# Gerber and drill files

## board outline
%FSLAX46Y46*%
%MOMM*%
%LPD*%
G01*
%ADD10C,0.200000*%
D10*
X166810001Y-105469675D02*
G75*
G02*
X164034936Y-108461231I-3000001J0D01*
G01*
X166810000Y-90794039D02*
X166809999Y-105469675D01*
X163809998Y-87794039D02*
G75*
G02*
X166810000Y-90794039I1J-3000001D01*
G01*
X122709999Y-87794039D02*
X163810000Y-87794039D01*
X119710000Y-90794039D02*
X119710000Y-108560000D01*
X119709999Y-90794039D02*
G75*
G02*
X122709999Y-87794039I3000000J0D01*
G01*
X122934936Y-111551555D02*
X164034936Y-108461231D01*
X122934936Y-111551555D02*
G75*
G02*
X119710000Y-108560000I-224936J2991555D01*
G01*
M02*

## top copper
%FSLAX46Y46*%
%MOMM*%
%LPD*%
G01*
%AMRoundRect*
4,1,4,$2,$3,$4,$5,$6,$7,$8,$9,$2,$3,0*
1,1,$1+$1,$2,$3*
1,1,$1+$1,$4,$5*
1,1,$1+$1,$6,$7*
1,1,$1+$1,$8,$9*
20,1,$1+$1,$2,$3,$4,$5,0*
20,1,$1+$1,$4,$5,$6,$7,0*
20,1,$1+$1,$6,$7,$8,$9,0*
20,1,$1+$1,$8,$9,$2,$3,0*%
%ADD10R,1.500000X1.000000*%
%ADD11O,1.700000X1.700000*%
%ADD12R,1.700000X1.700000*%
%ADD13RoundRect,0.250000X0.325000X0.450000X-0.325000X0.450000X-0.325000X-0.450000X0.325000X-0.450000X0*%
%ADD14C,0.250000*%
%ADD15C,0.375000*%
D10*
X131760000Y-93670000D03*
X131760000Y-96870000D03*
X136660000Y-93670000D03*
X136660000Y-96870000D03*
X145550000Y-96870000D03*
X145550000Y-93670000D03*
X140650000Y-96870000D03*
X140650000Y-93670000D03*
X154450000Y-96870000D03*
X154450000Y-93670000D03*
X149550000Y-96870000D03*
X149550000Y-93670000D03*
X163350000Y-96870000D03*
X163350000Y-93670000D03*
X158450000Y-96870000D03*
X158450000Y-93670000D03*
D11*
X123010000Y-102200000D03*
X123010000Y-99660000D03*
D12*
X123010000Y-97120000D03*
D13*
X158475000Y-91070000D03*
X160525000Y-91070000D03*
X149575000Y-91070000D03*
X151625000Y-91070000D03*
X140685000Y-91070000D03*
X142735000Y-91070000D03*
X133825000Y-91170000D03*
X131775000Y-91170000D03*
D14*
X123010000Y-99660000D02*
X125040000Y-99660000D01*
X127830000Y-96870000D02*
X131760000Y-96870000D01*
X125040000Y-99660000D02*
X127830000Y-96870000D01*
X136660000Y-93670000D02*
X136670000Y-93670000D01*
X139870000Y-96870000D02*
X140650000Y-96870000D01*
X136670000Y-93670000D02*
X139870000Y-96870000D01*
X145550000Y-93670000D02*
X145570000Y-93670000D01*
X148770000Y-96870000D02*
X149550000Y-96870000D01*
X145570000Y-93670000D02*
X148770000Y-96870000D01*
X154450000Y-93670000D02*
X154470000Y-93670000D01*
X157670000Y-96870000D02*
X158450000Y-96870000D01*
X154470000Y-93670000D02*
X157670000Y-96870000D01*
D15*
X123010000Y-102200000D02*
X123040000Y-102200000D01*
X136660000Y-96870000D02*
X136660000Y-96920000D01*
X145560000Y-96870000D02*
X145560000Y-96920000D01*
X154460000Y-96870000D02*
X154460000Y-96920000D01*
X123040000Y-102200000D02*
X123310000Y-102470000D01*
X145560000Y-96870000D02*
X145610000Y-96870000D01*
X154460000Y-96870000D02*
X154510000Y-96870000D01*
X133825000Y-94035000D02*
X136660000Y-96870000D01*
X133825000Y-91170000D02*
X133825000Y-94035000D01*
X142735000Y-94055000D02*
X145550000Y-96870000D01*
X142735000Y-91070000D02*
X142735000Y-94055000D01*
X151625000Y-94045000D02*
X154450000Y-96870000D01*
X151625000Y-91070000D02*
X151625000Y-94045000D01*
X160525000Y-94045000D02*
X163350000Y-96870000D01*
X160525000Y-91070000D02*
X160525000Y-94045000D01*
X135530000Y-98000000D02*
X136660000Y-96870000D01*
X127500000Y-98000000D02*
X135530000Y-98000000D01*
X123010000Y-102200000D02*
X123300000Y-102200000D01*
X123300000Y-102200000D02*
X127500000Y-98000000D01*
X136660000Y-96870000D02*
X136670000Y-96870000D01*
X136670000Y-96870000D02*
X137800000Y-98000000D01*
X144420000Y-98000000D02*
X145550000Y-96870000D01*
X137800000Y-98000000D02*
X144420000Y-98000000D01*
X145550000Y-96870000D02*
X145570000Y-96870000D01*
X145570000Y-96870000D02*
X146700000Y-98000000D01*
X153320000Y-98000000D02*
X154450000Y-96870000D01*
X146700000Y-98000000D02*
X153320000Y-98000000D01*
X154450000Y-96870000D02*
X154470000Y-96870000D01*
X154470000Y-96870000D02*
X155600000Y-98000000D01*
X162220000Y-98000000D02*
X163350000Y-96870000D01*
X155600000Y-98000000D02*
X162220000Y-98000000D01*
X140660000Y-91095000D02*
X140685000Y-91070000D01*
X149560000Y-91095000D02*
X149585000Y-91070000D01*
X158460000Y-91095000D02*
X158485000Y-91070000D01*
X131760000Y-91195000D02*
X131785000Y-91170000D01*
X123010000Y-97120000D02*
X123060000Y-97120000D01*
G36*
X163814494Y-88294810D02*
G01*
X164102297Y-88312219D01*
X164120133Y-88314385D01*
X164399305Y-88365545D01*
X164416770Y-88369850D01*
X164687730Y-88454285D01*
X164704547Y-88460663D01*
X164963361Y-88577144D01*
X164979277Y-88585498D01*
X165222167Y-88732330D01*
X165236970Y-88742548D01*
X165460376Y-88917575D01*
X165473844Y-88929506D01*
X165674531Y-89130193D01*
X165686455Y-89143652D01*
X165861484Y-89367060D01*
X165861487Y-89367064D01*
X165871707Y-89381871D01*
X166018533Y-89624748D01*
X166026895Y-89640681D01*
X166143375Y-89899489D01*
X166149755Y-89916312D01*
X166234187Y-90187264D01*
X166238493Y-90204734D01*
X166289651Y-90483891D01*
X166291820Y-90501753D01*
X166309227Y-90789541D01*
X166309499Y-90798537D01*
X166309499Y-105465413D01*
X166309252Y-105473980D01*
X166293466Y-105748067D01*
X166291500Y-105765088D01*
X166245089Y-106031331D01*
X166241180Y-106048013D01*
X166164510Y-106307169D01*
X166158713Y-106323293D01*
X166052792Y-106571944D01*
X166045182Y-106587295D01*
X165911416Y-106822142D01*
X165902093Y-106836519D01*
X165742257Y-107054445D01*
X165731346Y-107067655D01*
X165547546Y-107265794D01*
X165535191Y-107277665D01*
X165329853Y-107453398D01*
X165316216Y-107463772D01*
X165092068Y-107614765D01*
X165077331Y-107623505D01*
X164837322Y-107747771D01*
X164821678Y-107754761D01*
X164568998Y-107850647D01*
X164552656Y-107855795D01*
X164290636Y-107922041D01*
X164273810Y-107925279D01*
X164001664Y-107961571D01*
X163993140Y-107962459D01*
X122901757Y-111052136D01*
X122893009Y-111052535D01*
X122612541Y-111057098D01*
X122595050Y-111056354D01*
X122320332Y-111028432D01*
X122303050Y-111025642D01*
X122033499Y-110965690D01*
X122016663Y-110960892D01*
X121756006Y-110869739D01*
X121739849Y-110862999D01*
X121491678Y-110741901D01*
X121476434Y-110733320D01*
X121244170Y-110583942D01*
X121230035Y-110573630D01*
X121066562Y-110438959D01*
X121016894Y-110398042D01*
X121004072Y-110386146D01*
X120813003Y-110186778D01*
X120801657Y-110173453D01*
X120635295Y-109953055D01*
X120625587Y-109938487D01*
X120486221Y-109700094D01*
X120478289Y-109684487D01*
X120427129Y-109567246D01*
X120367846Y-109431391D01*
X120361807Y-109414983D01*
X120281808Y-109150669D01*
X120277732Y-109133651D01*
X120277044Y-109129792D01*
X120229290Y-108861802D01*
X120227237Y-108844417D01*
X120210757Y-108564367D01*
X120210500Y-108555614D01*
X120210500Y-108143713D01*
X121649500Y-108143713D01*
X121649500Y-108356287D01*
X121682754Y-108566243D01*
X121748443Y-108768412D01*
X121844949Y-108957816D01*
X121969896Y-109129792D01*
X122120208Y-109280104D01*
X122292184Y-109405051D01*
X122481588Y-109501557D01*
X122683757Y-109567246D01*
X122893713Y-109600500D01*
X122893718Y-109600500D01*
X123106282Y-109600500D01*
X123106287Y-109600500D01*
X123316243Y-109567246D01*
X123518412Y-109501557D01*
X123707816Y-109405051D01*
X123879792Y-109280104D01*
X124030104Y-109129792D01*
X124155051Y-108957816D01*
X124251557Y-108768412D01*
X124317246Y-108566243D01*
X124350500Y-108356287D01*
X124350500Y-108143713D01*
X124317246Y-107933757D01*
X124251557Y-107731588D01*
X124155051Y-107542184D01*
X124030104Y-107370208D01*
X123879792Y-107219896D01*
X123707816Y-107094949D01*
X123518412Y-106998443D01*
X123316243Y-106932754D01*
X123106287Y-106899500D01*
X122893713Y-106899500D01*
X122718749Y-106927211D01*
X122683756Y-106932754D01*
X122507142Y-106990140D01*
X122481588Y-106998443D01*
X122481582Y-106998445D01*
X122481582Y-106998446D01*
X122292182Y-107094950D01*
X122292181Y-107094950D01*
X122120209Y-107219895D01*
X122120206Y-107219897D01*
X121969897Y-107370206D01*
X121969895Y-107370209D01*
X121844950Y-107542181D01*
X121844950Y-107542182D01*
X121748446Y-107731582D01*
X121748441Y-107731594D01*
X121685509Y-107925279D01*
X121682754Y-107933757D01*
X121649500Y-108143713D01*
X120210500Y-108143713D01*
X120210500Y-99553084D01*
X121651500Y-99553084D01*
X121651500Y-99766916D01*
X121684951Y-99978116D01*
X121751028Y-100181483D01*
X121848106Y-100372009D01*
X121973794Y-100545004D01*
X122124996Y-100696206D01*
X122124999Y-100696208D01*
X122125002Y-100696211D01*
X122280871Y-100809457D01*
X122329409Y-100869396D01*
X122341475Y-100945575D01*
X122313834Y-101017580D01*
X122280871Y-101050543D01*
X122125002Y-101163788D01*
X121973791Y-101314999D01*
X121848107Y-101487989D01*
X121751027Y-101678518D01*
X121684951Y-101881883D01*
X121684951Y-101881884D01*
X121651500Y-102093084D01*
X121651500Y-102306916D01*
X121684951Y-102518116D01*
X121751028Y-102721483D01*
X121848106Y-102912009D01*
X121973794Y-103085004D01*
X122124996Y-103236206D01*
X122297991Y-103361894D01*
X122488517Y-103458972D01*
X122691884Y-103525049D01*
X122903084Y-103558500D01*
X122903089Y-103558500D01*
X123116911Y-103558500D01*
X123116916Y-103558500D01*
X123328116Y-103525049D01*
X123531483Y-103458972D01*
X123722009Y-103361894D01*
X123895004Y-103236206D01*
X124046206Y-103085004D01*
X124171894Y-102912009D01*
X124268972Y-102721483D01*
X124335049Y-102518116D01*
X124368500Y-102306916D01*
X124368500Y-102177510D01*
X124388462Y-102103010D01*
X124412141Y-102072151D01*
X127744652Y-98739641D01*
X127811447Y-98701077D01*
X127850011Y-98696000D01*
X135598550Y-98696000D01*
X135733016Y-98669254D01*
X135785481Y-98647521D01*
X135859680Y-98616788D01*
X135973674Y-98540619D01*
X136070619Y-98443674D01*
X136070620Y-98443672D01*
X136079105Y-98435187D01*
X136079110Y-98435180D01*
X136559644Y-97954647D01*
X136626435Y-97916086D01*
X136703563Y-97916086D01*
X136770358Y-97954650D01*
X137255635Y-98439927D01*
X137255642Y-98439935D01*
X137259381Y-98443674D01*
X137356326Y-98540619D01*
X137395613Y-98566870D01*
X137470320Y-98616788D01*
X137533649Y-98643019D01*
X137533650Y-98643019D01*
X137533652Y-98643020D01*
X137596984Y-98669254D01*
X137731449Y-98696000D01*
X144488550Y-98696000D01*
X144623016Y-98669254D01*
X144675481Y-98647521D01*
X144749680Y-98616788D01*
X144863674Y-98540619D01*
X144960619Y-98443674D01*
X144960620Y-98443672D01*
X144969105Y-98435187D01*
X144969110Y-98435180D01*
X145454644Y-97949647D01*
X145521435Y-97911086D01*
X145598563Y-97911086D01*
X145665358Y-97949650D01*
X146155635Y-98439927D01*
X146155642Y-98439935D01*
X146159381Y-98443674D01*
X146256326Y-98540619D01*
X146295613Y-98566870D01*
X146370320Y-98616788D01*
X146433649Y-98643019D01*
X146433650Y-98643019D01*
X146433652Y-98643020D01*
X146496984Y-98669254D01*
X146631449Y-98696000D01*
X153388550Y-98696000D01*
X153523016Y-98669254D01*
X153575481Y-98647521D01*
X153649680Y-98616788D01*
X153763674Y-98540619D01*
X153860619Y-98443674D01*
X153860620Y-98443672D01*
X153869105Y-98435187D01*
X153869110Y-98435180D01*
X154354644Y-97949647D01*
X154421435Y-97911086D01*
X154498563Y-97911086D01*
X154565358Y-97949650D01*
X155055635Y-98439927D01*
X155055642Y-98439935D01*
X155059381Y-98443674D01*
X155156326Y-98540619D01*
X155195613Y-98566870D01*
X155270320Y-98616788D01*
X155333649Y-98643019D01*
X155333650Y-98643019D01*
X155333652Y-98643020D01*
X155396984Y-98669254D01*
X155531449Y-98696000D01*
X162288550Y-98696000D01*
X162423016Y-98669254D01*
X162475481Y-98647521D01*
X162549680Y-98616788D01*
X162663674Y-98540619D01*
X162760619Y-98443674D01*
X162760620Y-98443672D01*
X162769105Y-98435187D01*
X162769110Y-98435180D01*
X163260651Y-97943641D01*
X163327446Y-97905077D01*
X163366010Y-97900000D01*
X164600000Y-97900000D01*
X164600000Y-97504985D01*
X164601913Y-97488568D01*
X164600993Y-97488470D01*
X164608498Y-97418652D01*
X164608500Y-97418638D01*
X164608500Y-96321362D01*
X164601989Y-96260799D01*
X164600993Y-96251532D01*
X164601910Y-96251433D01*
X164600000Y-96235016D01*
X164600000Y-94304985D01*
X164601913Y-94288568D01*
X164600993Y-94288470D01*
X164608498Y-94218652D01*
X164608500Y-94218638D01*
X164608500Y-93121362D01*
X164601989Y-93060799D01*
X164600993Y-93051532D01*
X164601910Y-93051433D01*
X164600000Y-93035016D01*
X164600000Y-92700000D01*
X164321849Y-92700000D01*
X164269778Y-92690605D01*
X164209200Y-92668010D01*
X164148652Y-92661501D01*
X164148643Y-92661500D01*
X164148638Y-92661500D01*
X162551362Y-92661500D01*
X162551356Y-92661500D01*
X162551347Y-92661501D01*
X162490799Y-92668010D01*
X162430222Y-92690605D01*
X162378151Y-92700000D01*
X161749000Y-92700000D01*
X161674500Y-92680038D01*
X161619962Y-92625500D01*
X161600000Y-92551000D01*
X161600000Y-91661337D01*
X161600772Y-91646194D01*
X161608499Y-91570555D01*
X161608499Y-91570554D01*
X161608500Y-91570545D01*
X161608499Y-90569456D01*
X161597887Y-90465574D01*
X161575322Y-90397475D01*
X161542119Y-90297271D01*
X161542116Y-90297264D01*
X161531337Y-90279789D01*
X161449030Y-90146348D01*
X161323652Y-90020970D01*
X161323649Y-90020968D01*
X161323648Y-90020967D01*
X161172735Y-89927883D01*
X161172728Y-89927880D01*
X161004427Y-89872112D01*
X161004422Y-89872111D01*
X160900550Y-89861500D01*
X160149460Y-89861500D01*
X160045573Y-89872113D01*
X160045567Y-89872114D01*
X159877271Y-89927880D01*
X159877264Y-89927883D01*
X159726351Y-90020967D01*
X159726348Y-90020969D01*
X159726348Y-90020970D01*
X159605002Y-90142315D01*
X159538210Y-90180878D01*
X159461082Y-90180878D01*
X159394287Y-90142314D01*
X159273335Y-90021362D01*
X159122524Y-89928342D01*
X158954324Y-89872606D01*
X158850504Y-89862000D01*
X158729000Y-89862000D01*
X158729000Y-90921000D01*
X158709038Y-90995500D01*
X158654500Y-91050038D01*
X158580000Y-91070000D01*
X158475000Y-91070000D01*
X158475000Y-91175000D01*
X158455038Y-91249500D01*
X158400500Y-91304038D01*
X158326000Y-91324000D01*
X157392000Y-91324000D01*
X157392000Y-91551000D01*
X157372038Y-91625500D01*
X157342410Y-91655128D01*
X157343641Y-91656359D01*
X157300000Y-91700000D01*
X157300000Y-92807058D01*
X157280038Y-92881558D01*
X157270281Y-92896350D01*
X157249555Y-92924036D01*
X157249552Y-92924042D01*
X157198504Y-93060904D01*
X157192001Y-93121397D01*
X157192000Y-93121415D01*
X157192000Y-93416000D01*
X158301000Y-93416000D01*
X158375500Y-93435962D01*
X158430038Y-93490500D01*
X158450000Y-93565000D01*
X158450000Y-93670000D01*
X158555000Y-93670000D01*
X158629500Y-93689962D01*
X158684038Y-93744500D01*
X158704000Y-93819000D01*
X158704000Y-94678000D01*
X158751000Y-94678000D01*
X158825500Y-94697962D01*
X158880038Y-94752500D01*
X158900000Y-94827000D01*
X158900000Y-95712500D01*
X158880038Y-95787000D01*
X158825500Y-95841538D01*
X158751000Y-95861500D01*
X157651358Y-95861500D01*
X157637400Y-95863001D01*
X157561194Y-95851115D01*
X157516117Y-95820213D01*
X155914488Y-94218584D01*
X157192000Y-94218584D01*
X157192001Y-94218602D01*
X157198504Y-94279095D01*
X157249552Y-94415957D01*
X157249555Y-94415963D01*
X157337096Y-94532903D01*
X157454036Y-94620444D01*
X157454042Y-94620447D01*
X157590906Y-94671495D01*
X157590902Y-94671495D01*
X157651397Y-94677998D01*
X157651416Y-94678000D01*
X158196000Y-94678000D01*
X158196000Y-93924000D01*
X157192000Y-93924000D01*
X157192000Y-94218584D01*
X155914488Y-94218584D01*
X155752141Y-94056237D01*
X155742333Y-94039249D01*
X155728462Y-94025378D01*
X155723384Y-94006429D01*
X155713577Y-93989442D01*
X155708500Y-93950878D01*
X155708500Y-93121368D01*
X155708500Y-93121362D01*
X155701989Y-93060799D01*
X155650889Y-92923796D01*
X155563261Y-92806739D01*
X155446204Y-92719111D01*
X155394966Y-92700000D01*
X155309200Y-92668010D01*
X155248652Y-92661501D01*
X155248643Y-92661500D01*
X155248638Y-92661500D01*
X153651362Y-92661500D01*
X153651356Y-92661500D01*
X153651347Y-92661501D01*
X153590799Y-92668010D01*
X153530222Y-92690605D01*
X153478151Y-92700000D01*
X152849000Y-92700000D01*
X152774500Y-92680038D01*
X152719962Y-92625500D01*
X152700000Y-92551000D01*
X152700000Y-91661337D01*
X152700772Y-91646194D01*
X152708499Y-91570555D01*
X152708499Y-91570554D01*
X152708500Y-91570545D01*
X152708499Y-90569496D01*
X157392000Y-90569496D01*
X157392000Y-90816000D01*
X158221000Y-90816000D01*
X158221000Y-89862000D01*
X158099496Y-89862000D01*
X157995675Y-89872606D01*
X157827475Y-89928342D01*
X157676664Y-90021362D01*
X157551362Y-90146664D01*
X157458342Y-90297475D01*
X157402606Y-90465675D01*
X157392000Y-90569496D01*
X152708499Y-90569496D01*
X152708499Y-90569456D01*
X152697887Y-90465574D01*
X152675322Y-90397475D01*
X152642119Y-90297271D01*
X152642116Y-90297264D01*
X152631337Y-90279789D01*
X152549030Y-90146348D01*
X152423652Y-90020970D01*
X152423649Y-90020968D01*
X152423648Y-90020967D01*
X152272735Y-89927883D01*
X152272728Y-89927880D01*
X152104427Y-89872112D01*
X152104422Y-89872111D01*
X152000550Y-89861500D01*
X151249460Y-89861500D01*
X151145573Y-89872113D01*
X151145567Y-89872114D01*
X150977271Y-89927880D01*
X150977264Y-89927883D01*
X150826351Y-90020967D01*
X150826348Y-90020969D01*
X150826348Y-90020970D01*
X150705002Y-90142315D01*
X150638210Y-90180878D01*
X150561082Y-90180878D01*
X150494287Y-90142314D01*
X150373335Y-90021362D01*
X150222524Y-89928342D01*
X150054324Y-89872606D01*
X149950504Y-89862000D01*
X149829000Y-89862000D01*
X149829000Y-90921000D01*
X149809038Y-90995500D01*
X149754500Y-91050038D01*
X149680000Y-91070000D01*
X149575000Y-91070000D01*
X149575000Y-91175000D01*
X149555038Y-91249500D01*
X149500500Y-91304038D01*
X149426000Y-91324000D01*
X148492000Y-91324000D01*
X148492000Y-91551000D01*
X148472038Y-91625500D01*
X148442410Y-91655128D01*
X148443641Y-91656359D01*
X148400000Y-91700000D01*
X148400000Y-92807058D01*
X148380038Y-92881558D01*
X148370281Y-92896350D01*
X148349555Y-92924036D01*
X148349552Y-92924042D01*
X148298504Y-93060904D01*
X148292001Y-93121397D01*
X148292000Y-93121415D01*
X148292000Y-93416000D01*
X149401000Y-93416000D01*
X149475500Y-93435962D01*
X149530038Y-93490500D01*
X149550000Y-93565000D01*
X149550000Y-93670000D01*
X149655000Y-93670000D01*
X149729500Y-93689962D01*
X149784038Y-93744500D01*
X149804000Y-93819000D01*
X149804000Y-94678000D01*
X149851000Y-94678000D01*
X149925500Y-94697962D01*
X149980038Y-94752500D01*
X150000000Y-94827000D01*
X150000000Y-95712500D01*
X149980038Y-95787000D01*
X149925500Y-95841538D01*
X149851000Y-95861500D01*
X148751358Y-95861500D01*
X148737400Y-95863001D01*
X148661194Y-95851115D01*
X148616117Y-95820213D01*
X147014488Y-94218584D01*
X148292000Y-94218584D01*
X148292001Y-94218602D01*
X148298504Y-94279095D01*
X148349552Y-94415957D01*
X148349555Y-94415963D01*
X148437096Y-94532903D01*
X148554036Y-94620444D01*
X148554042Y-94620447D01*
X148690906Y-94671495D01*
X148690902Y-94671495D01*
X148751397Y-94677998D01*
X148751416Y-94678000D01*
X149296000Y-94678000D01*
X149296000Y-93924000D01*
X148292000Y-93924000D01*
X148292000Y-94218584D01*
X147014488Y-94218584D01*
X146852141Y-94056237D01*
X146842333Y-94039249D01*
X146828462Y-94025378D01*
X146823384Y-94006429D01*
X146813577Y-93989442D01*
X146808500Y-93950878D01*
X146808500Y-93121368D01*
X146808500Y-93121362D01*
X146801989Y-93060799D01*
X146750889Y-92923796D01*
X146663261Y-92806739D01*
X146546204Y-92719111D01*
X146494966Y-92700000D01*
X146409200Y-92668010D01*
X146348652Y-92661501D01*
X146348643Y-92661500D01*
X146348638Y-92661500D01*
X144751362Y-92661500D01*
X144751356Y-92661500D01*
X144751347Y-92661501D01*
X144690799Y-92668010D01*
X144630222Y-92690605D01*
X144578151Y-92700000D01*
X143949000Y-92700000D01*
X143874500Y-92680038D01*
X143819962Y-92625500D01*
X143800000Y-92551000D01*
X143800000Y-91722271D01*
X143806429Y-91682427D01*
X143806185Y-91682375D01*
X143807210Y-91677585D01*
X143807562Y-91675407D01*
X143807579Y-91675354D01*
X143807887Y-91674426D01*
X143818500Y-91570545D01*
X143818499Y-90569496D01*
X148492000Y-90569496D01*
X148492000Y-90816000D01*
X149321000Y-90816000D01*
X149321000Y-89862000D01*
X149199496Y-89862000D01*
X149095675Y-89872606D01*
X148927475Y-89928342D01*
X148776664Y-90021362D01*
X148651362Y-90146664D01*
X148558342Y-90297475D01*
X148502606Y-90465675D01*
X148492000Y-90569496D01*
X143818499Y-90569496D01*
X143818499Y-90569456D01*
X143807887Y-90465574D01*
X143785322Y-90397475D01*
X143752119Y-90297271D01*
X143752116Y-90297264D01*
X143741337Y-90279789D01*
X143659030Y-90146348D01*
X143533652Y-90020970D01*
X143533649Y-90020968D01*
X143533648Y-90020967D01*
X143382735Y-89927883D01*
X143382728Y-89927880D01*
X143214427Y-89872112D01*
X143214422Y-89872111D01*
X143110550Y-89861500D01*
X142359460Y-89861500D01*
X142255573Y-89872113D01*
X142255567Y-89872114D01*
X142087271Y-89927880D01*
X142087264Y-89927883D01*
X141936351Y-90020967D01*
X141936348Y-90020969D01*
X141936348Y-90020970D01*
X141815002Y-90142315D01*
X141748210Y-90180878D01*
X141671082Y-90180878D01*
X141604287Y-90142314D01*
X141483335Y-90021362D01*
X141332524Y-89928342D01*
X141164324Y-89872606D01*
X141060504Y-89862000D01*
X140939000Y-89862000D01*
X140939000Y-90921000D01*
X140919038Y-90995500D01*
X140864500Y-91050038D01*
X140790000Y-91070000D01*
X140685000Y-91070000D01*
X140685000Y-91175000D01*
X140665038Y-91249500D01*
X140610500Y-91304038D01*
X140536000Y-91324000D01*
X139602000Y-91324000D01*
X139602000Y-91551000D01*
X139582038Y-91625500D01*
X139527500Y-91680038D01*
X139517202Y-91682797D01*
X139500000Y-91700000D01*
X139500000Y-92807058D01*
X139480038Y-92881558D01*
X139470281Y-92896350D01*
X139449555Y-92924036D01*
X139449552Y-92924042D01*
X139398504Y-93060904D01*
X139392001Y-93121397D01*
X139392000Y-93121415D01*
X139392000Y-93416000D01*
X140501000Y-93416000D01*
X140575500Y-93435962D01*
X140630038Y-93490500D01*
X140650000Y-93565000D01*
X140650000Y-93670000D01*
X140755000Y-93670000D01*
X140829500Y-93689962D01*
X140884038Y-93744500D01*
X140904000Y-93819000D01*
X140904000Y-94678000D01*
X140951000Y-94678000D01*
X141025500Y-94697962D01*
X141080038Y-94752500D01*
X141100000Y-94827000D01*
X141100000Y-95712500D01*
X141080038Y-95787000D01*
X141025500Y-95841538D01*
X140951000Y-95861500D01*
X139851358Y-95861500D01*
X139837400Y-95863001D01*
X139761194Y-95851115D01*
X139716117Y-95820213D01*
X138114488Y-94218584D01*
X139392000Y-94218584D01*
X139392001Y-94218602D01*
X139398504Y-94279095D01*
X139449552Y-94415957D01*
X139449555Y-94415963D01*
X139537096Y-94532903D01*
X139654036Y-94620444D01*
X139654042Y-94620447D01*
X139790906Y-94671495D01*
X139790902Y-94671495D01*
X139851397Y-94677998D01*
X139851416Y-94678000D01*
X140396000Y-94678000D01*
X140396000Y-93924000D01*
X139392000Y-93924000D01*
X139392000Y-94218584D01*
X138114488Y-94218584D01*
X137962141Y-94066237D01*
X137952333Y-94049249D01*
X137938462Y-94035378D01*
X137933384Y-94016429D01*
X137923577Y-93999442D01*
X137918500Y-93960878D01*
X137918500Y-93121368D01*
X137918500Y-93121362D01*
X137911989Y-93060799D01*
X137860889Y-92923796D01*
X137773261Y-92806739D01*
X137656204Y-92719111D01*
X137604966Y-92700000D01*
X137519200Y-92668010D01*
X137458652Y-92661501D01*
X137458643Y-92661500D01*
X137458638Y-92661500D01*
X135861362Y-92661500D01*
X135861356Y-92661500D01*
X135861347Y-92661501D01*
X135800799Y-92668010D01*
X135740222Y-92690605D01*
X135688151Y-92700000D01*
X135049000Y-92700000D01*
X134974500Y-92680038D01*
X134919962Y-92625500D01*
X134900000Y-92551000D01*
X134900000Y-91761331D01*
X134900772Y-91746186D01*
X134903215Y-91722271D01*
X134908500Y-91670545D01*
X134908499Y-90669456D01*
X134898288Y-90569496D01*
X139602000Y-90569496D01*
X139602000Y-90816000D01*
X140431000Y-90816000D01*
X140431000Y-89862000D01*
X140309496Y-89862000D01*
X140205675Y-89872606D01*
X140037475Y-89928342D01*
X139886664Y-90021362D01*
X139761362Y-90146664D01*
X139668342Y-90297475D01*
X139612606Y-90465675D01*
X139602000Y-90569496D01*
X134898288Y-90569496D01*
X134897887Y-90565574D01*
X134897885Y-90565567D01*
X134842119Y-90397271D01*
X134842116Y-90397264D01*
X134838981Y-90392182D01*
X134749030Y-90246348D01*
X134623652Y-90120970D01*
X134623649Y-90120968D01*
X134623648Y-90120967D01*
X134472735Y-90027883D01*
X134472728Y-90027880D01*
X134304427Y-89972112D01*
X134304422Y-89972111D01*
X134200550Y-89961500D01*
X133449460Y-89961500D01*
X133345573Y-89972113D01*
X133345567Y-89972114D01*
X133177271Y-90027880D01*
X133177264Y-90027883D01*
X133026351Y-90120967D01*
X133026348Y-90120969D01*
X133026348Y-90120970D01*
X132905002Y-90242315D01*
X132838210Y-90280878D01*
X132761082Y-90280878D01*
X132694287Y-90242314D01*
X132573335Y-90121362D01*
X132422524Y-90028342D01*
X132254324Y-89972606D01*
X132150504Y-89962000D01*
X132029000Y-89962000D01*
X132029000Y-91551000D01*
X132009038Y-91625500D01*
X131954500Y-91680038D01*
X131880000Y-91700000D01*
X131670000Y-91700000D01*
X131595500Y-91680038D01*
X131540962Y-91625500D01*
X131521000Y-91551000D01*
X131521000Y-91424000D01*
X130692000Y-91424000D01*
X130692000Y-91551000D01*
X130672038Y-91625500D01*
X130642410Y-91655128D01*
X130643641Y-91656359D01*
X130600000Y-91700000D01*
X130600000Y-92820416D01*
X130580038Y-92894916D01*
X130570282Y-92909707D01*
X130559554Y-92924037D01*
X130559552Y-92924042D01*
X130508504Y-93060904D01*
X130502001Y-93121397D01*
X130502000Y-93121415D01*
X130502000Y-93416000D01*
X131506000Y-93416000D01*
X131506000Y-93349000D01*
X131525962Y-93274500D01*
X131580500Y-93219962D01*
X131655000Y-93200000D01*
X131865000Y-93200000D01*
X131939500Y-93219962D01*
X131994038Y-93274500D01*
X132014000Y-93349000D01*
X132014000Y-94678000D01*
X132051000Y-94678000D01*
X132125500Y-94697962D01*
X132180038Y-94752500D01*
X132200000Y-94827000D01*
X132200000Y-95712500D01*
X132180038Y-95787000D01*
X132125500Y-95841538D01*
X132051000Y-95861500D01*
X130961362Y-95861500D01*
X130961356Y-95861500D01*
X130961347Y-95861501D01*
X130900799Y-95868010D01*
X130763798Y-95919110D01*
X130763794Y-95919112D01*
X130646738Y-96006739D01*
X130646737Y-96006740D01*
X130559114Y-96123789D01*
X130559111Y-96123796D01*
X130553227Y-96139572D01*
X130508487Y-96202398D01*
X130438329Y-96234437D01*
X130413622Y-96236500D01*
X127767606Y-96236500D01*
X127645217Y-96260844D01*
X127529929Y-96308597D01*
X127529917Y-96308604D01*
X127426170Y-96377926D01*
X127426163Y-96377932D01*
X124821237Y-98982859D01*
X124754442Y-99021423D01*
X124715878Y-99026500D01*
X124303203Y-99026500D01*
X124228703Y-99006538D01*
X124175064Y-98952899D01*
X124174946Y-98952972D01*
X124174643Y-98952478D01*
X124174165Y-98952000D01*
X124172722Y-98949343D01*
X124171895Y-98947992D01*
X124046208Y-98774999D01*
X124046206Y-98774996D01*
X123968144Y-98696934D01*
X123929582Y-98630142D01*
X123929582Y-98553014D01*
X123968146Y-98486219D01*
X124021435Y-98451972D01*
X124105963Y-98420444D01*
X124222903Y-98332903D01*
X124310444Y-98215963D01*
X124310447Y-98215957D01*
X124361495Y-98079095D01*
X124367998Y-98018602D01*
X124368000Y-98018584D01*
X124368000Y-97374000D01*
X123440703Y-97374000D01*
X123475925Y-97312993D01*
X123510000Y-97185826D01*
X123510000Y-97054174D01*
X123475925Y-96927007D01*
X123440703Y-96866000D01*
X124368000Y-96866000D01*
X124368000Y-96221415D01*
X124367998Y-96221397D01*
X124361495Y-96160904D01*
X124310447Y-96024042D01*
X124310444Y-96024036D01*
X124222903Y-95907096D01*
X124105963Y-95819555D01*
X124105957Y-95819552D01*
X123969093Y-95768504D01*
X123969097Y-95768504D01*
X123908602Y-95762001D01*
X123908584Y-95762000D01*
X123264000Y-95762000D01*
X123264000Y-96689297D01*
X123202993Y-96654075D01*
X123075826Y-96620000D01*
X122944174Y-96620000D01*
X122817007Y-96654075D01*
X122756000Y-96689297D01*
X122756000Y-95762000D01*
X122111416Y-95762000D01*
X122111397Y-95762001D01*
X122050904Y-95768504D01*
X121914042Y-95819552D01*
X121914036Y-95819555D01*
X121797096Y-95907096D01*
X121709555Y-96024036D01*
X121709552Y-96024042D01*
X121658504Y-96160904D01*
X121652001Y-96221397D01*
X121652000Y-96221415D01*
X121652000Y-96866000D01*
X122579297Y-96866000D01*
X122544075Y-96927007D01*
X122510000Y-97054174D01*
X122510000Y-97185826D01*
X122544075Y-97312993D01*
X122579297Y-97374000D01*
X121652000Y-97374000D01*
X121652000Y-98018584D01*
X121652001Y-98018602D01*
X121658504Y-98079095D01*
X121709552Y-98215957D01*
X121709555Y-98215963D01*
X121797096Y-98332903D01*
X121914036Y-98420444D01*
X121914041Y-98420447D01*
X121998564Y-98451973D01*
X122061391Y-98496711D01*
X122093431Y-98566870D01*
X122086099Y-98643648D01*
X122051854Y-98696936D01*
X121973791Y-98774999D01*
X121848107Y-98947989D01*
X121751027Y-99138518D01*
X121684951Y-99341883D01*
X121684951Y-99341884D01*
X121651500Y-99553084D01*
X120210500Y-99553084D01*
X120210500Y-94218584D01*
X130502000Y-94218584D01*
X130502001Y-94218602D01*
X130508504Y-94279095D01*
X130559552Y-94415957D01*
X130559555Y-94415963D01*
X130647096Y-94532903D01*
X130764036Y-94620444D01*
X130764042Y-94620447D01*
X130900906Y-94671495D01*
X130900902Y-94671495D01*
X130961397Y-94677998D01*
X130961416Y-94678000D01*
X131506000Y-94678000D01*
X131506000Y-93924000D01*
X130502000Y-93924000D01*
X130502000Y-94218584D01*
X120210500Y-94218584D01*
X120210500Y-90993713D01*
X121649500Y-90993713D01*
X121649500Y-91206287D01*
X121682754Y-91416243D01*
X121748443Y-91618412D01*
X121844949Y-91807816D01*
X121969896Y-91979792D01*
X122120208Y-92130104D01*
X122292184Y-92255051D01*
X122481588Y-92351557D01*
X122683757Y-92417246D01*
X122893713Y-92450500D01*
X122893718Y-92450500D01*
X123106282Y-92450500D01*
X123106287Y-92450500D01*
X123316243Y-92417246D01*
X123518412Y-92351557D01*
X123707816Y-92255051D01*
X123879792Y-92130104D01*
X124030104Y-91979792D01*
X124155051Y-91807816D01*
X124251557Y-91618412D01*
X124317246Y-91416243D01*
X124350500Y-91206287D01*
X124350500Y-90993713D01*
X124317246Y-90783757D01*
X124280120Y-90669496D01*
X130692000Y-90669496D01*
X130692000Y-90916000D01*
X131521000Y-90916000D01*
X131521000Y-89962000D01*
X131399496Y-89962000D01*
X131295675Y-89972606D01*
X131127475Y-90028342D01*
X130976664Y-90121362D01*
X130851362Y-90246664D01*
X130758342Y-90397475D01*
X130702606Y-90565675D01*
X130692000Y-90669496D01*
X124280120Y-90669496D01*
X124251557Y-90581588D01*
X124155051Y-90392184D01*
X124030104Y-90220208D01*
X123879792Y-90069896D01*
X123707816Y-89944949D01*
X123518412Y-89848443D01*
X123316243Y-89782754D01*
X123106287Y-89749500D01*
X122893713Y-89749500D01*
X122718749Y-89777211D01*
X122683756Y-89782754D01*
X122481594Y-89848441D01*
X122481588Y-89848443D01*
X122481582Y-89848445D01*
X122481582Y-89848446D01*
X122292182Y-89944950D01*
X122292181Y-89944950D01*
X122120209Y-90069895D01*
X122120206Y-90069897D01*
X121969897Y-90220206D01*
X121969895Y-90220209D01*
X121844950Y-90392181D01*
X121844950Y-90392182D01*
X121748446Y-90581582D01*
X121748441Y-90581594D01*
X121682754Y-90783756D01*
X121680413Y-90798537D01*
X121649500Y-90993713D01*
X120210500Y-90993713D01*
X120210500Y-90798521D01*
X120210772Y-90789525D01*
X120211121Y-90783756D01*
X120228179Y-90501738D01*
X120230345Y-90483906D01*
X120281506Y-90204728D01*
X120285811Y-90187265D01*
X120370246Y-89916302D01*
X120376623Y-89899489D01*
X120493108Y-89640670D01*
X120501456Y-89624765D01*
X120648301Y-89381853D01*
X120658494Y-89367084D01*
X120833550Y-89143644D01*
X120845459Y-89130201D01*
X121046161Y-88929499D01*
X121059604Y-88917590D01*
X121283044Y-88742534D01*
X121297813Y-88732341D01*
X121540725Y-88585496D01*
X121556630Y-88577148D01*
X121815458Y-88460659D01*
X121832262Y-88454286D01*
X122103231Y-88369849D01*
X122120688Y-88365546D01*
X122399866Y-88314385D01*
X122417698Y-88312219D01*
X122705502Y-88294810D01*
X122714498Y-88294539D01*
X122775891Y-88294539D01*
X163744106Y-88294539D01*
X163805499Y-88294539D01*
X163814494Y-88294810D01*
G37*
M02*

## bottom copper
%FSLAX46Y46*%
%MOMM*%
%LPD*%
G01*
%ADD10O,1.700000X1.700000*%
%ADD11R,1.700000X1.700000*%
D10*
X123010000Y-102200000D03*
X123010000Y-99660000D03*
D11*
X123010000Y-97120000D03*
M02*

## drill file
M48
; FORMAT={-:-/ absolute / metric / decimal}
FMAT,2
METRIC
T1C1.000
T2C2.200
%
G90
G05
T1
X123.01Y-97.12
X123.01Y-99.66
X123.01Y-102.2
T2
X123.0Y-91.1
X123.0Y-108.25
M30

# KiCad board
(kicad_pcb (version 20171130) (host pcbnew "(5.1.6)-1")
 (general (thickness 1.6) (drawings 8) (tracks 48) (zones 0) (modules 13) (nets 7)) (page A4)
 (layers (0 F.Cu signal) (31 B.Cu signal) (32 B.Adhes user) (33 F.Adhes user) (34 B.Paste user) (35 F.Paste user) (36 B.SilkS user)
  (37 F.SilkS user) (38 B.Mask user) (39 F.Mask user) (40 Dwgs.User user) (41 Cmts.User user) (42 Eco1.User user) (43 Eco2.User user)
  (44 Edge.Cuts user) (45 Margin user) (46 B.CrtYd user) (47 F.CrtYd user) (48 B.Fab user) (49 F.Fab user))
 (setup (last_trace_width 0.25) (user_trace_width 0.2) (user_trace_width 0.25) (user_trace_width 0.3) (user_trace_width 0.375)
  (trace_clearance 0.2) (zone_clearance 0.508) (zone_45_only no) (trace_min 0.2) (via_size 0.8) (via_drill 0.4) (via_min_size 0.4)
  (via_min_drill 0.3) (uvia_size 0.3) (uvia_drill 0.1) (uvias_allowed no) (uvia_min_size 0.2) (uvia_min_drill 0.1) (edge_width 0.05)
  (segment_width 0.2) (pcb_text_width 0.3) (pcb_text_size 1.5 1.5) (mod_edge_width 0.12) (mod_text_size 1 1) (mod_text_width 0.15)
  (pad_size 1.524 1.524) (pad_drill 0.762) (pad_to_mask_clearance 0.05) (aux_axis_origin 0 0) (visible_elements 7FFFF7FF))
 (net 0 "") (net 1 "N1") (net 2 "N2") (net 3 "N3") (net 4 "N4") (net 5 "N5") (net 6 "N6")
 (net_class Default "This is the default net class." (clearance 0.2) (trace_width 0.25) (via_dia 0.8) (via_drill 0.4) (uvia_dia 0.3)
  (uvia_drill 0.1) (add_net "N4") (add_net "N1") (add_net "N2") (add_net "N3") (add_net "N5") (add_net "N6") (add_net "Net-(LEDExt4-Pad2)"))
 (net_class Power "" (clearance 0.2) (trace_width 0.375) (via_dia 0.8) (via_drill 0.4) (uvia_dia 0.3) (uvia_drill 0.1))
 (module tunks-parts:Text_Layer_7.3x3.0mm (layer F.Cu) (at 152 102.7 270)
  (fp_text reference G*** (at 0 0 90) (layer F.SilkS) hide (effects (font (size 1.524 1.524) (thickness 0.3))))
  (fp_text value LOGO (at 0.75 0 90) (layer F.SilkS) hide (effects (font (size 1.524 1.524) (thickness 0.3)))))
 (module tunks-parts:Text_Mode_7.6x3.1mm (layer F.Cu) (at 160.9 102.8 270)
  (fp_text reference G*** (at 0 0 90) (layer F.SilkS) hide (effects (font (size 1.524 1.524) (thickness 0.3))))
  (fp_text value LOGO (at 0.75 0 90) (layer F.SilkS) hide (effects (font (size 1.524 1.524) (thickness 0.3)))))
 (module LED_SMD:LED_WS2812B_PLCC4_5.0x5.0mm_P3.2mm (layer F.Cu) (at 134.21 95.27 180)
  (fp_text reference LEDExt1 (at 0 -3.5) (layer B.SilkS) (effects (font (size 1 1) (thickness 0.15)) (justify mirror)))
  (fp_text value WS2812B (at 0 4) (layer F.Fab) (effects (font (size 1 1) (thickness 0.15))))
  (pad 3 smd rect (at 2.45 1.6 180) (size 1.5 1) (layers F.Cu F.Paste F.Mask) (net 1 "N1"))
  (pad 4 smd rect (at 2.45 -1.6 180) (size 1.5 1) (layers F.Cu F.Paste F.Mask) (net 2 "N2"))
  (pad 2 smd rect (at -2.45 1.6 180) (size 1.5 1) (layers F.Cu F.Paste F.Mask) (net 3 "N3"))
  (pad 1 smd rect (at -2.45 -1.6 180) (size 1.5 1) (layers F.Cu F.Paste F.Mask) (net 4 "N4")))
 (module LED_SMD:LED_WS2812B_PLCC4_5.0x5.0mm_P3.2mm (layer F.Cu) (at 143.1 95.27 180)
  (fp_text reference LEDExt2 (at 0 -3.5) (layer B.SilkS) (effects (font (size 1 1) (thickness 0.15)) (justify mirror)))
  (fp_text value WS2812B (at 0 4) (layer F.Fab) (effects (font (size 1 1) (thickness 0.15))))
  (pad 1 smd rect (at -2.45 -1.6 180) (size 1.5 1) (layers F.Cu F.Paste F.Mask) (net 4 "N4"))
  (pad 2 smd rect (at -2.45 1.6 180) (size 1.5 1) (layers F.Cu F.Paste F.Mask) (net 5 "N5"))
  (pad 4 smd rect (at 2.45 -1.6 180) (size 1.5 1) (layers F.Cu F.Paste F.Mask) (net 3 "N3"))
  (pad 3 smd rect (at 2.45 1.6 180) (size 1.5 1) (layers F.Cu F.Paste F.Mask) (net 1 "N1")))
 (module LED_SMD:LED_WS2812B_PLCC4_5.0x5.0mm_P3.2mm (layer F.Cu) (at 152 95.27 180)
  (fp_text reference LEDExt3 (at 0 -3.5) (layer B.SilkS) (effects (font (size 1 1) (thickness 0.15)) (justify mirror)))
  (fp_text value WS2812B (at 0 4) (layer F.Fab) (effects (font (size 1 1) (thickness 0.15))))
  (pad 1 smd rect (at -2.45 -1.6 180) (size 1.5 1) (layers F.Cu F.Paste F.Mask) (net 4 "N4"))
  (pad 2 smd rect (at -2.45 1.6 180) (size 1.5 1) (layers F.Cu F.Paste F.Mask) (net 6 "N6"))
  (pad 4 smd rect (at 2.45 -1.6 180) (size 1.5 1) (layers F.Cu F.Paste F.Mask) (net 5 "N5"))
  (pad 3 smd rect (at 2.45 1.6 180) (size 1.5 1) (layers F.Cu F.Paste F.Mask) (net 1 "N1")))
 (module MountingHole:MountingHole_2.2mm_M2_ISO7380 (layer F.Cu) (at 123 108.25)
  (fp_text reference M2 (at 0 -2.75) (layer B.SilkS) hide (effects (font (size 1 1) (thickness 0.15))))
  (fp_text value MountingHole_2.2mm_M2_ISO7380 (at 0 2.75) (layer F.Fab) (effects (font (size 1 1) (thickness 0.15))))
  (pad 1 np_thru_hole circle (at 0 0) (size 2.2 2.2) (drill 2.2) (layers *.Cu *.Mask)))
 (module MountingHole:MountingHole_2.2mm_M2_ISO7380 (layer F.Cu) (at 123 91.1)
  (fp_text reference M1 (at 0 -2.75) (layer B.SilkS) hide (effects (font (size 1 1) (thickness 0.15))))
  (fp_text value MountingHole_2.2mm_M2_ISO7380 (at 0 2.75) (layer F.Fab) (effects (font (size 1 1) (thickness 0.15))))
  (pad 1 np_thru_hole circle (at 0 0) (size 2.2 2.2) (drill 2.2) (layers *.Cu *.Mask)))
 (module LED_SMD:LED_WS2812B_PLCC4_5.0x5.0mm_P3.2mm (layer F.Cu) (at 160.9 95.27 180)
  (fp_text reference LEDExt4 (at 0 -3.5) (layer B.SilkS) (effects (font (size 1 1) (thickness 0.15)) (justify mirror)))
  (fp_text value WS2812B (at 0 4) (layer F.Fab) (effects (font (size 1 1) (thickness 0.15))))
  (pad 1 smd rect (at -2.45 -1.6 180) (size 1.5 1) (layers F.Cu F.Paste F.Mask) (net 4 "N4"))
  (pad 2 smd rect (at -2.45 1.6 180) (size 1.5 1) (layers F.Cu F.Paste F.Mask))
  (pad 4 smd rect (at 2.45 -1.6 180) (size 1.5 1) (layers F.Cu F.Paste F.Mask) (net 6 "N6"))
  (pad 3 smd rect (at 2.45 1.6 180) (size 1.5 1) (layers F.Cu F.Paste F.Mask) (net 1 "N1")))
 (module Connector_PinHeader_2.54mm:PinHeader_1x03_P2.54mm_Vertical (layer B.Cu) (at 123.01 97.12 180)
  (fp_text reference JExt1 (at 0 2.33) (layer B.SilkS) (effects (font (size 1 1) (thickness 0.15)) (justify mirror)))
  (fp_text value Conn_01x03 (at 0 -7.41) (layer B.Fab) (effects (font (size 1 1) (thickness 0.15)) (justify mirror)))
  (pad 3 thru_hole oval (at 0 -5.08 180) (size 1.7 1.7) (drill 1) (layers *.Cu *.Mask) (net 4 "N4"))
  (pad 2 thru_hole oval (at 0 -2.54 180) (size 1.7 1.7) (drill 1) (layers *.Cu *.Mask) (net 2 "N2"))
  (pad 1 thru_hole rect (at 0 0 180) (size 1.7 1.7) (drill 1) (layers *.Cu *.Mask) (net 1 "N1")))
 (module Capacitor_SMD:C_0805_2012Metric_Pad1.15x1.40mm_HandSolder (layer F.Cu) (at 159.5 91.07 180)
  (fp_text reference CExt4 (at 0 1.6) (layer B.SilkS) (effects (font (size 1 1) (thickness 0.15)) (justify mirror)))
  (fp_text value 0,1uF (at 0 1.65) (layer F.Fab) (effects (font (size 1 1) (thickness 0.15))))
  (pad 2 smd roundrect (at 1.025 0 180) (size 1.15 1.4) (layers F.Cu F.Paste F.Mask) (roundrect_rratio 0.217391) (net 1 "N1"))
  (pad 1 smd roundrect (at -1.025 0 180) (size 1.15 1.4) (layers F.Cu F.Paste F.Mask) (roundrect_rratio 0.217391) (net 4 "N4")))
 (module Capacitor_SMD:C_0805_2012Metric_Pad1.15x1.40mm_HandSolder (layer F.Cu) (at 150.6 91.07 180)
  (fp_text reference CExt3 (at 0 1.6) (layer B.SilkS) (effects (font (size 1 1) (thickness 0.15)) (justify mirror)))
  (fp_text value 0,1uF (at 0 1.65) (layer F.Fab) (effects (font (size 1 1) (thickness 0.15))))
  (pad 2 smd roundrect (at 1.025 0 180) (size 1.15 1.4) (layers F.Cu F.Paste F.Mask) (roundrect_rratio 0.217391) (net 1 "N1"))
  (pad 1 smd roundrect (at -1.025 0 180) (size 1.15 1.4) (layers F.Cu F.Paste F.Mask) (roundrect_rratio 0.217391) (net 4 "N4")))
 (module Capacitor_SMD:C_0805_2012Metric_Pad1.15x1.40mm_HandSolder (layer F.Cu) (at 141.71 91.07 180)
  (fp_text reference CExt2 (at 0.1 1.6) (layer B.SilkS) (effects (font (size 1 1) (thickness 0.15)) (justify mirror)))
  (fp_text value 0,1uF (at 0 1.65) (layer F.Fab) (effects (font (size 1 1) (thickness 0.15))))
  (pad 2 smd roundrect (at 1.025 0 180) (size 1.15 1.4) (layers F.Cu F.Paste F.Mask) (roundrect_rratio 0.217391) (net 1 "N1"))
  (pad 1 smd roundrect (at -1.025 0 180) (size 1.15 1.4) (layers F.Cu F.Paste F.Mask) (roundrect_rratio 0.217391) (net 4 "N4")))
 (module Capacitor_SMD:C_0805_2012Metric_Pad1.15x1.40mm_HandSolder (layer F.Cu) (at 132.8 91.17 180)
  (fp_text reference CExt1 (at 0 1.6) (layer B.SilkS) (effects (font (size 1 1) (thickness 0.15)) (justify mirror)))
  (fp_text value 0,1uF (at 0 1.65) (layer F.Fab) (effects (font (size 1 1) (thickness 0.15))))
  (pad 1 smd roundrect (at -1.025 0 180) (size 1.15 1.4) (layers F.Cu F.Paste F.Mask) (roundrect_rratio 0.217391) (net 4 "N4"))
  (pad 2 smd roundrect (at 1.025 0 180) (size 1.15 1.4) (layers F.Cu F.Paste F.Mask) (roundrect_rratio 0.217391) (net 1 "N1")))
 (gr_arc (start 163.81 105.469675) (end 164.034936 108.461231) (angle -85.7) (layer Edge.Cuts) (width 0.2))
 (gr_line (start 166.81 90.794039) (end 166.809999 105.469675) (layer Edge.Cuts) (width 0.2))
 (gr_arc (start 163.809999 90.79404) (end 166.81 90.794039) (angle -90) (layer Edge.Cuts) (width 0.2))
 (gr_line (start 122.709999 87.794039) (end 163.81 87.794039) (layer Edge.Cuts) (width 0.2))
 (gr_line (start 119.71 90.794039) (end 119.71 108.56) (layer Edge.Cuts) (width 0.2))
 (gr_arc (start 122.709999 90.794039) (end 122.709999 87.794039) (angle -90) (layer Edge.Cuts) (width 0.2))
 (gr_line (start 122.934936 111.551555) (end 164.034936 108.461231) (layer Edge.Cuts) (width 0.2))
 (gr_arc (start 122.71 108.56) (end 119.71 108.56) (angle -94.3) (layer Edge.Cuts) (width 0.2))
 (segment (start 123.01 99.66) (end 125.04 99.66) (width 0.25) (layer F.Cu) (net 2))
 (segment (start 127.83 96.87) (end 131.76 96.87) (width 0.25) (layer F.Cu) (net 2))
 (segment (start 125.04 99.66) (end 127.83 96.87) (width 0.25) (layer F.Cu) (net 2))
 (segment (start 136.66 93.67) (end 136.67 93.67) (width 0.25) (layer F.Cu) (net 3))
 (segment (start 139.87 96.87) (end 140.65 96.87) (width 0.25) (layer F.Cu) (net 3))
 (segment (start 136.67 93.67) (end 139.87 96.87) (width 0.25) (layer F.Cu) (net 3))
 (segment (start 145.55 93.67) (end 145.57 93.67) (width 0.25) (layer F.Cu) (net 5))
 (segment (start 148.77 96.87) (end 149.55 96.87) (width 0.25) (layer F.Cu) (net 5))
 (segment (start 145.57 93.67) (end 148.77 96.87) (width 0.25) (layer F.Cu) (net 5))
 (segment (start 154.45 93.67) (end 154.47 93.67) (width 0.25) (layer F.Cu) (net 6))
 (segment (start 157.67 96.87) (end 158.45 96.87) (width 0.25) (layer F.Cu) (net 6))
 (segment (start 154.47 93.67) (end 157.67 96.87) (width 0.25) (layer F.Cu) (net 6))
 (segment (start 123.01 102.2) (end 123.04 102.2) (width 0.375) (layer F.Cu) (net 4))
 (segment (start 136.66 96.87) (end 136.66 96.92) (width 0.375) (layer F.Cu) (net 4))
 (segment (start 145.56 96.87) (end 145.56 96.92) (width 0.375) (layer F.Cu) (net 4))
 (segment (start 154.46 96.87) (end 154.46 96.92) (width 0.375) (layer F.Cu) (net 4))
 (segment (start 123.04 102.2) (end 123.31 102.47) (width 0.375) (layer F.Cu) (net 4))
 (segment (start 145.56 96.87) (end 145.61 96.87) (width 0.375) (layer F.Cu) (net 4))
 (segment (start 154.46 96.87) (end 154.51 96.87) (width 0.375) (layer F.Cu) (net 4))
 (segment (start 133.825 94.035) (end 136.66 96.87) (width 0.375) (layer F.Cu) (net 4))
 (segment (start 133.825 91.17) (end 133.825 94.035) (width 0.375) (layer F.Cu) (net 4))
 (segment (start 142.735 94.055) (end 145.55 96.87) (width 0.375) (layer F.Cu) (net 4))
 (segment (start 142.735 91.07) (end 142.735 94.055) (width 0.375) (layer F.Cu) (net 4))
 (segment (start 151.625 94.045) (end 154.45 96.87) (width 0.375) (layer F.Cu) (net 4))
 (segment (start 151.625 91.07) (end 151.625 94.045) (width 0.375) (layer F.Cu) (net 4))
 (segment (start 160.525 94.045) (end 163.35 96.87) (width 0.375) (layer F.Cu) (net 4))
 (segment (start 160.525 91.07) (end 160.525 94.045) (width 0.375) (layer F.Cu) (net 4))
 (segment (start 135.53 98) (end 136.66 96.87) (width 0.375) (layer F.Cu) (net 4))
 (segment (start 127.5 98) (end 135.53 98) (width 0.375) (layer F.Cu) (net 4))
 (segment (start 123.01 102.2) (end 123.3 102.2) (width 0.375) (layer F.Cu) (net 4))
 (segment (start 123.3 102.2) (end 127.5 98) (width 0.375) (layer F.Cu) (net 4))
 (segment (start 136.66 96.87) (end 136.67 96.87) (width 0.375) (layer F.Cu) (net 4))
 (segment (start 136.67 96.87) (end 137.8 98) (width 0.375) (layer F.Cu) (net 4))
 (segment (start 144.42 98) (end 145.55 96.87) (width 0.375) (layer F.Cu) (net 4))
 (segment (start 137.8 98) (end 144.42 98) (width 0.375) (layer F.Cu) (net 4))
 (segment (start 145.55 96.87) (end 145.57 96.87) (width 0.375) (layer F.Cu) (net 4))
 (segment (start 145.57 96.87) (end 146.7 98) (width 0.375) (layer F.Cu) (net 4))
 (segment (start 153.32 98) (end 154.45 96.87) (width 0.375) (layer F.Cu) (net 4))
 (segment (start 146.7 98) (end 153.32 98) (width 0.375) (layer F.Cu) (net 4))
 (segment (start 154.45 96.87) (end 154.47 96.87) (width 0.375) (layer F.Cu) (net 4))
 (segment (start 154.47 96.87) (end 155.6 98) (width 0.375) (layer F.Cu) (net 4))
 (segment (start 162.22 98) (end 163.35 96.87) (width 0.375) (layer F.Cu) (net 4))
 (segment (start 155.6 98) (end 162.22 98) (width 0.375) (layer F.Cu) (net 4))
 (segment (start 140.66 91.095) (end 140.685 91.07) (width 0.375) (layer F.Cu) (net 1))
 (segment (start 149.56 91.095) (end 149.585 91.07) (width 0.375) (layer F.Cu) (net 1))
 (segment (start 158.46 91.095) (end 158.485 91.07) (width 0.375) (layer F.Cu) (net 1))
 (segment (start 131.76 91.195) (end 131.785 91.17) (width 0.375) (layer F.Cu) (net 1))
 (segment (start 123.01 97.12) (end 123.06 97.12) (width 0.375) (layer F.Cu) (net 1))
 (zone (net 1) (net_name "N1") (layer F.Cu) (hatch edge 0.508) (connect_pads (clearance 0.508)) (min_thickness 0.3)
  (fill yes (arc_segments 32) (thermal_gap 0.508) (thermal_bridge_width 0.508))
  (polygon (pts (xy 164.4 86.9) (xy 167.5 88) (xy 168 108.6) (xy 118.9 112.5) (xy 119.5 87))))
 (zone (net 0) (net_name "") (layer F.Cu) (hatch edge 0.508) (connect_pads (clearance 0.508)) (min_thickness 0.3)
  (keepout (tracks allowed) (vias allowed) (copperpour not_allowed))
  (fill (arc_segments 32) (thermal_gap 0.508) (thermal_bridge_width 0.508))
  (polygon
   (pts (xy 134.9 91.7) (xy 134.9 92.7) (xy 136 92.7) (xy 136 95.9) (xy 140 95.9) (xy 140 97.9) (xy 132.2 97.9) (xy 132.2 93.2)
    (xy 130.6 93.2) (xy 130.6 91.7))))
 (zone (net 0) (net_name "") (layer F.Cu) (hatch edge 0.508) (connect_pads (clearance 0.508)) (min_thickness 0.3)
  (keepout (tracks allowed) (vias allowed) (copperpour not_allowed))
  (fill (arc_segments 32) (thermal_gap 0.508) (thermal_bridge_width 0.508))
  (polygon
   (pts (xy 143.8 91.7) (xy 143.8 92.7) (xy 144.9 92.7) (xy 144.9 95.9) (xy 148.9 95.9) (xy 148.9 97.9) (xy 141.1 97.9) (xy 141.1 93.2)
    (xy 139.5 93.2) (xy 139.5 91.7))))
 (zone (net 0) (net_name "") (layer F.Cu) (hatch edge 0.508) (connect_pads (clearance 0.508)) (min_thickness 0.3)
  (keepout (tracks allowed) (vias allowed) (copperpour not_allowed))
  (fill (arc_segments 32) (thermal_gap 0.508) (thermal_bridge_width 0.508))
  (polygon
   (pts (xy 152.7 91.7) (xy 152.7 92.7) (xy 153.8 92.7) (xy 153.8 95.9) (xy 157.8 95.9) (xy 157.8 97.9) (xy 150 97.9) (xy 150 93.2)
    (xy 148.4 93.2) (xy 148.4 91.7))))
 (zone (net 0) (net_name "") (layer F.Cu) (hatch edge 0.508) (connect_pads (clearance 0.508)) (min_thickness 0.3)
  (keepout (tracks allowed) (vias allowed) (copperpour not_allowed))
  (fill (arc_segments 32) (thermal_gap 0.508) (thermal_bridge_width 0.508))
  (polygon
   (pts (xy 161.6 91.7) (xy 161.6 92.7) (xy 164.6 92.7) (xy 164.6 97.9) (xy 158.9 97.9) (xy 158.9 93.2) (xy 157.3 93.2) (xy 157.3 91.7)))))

